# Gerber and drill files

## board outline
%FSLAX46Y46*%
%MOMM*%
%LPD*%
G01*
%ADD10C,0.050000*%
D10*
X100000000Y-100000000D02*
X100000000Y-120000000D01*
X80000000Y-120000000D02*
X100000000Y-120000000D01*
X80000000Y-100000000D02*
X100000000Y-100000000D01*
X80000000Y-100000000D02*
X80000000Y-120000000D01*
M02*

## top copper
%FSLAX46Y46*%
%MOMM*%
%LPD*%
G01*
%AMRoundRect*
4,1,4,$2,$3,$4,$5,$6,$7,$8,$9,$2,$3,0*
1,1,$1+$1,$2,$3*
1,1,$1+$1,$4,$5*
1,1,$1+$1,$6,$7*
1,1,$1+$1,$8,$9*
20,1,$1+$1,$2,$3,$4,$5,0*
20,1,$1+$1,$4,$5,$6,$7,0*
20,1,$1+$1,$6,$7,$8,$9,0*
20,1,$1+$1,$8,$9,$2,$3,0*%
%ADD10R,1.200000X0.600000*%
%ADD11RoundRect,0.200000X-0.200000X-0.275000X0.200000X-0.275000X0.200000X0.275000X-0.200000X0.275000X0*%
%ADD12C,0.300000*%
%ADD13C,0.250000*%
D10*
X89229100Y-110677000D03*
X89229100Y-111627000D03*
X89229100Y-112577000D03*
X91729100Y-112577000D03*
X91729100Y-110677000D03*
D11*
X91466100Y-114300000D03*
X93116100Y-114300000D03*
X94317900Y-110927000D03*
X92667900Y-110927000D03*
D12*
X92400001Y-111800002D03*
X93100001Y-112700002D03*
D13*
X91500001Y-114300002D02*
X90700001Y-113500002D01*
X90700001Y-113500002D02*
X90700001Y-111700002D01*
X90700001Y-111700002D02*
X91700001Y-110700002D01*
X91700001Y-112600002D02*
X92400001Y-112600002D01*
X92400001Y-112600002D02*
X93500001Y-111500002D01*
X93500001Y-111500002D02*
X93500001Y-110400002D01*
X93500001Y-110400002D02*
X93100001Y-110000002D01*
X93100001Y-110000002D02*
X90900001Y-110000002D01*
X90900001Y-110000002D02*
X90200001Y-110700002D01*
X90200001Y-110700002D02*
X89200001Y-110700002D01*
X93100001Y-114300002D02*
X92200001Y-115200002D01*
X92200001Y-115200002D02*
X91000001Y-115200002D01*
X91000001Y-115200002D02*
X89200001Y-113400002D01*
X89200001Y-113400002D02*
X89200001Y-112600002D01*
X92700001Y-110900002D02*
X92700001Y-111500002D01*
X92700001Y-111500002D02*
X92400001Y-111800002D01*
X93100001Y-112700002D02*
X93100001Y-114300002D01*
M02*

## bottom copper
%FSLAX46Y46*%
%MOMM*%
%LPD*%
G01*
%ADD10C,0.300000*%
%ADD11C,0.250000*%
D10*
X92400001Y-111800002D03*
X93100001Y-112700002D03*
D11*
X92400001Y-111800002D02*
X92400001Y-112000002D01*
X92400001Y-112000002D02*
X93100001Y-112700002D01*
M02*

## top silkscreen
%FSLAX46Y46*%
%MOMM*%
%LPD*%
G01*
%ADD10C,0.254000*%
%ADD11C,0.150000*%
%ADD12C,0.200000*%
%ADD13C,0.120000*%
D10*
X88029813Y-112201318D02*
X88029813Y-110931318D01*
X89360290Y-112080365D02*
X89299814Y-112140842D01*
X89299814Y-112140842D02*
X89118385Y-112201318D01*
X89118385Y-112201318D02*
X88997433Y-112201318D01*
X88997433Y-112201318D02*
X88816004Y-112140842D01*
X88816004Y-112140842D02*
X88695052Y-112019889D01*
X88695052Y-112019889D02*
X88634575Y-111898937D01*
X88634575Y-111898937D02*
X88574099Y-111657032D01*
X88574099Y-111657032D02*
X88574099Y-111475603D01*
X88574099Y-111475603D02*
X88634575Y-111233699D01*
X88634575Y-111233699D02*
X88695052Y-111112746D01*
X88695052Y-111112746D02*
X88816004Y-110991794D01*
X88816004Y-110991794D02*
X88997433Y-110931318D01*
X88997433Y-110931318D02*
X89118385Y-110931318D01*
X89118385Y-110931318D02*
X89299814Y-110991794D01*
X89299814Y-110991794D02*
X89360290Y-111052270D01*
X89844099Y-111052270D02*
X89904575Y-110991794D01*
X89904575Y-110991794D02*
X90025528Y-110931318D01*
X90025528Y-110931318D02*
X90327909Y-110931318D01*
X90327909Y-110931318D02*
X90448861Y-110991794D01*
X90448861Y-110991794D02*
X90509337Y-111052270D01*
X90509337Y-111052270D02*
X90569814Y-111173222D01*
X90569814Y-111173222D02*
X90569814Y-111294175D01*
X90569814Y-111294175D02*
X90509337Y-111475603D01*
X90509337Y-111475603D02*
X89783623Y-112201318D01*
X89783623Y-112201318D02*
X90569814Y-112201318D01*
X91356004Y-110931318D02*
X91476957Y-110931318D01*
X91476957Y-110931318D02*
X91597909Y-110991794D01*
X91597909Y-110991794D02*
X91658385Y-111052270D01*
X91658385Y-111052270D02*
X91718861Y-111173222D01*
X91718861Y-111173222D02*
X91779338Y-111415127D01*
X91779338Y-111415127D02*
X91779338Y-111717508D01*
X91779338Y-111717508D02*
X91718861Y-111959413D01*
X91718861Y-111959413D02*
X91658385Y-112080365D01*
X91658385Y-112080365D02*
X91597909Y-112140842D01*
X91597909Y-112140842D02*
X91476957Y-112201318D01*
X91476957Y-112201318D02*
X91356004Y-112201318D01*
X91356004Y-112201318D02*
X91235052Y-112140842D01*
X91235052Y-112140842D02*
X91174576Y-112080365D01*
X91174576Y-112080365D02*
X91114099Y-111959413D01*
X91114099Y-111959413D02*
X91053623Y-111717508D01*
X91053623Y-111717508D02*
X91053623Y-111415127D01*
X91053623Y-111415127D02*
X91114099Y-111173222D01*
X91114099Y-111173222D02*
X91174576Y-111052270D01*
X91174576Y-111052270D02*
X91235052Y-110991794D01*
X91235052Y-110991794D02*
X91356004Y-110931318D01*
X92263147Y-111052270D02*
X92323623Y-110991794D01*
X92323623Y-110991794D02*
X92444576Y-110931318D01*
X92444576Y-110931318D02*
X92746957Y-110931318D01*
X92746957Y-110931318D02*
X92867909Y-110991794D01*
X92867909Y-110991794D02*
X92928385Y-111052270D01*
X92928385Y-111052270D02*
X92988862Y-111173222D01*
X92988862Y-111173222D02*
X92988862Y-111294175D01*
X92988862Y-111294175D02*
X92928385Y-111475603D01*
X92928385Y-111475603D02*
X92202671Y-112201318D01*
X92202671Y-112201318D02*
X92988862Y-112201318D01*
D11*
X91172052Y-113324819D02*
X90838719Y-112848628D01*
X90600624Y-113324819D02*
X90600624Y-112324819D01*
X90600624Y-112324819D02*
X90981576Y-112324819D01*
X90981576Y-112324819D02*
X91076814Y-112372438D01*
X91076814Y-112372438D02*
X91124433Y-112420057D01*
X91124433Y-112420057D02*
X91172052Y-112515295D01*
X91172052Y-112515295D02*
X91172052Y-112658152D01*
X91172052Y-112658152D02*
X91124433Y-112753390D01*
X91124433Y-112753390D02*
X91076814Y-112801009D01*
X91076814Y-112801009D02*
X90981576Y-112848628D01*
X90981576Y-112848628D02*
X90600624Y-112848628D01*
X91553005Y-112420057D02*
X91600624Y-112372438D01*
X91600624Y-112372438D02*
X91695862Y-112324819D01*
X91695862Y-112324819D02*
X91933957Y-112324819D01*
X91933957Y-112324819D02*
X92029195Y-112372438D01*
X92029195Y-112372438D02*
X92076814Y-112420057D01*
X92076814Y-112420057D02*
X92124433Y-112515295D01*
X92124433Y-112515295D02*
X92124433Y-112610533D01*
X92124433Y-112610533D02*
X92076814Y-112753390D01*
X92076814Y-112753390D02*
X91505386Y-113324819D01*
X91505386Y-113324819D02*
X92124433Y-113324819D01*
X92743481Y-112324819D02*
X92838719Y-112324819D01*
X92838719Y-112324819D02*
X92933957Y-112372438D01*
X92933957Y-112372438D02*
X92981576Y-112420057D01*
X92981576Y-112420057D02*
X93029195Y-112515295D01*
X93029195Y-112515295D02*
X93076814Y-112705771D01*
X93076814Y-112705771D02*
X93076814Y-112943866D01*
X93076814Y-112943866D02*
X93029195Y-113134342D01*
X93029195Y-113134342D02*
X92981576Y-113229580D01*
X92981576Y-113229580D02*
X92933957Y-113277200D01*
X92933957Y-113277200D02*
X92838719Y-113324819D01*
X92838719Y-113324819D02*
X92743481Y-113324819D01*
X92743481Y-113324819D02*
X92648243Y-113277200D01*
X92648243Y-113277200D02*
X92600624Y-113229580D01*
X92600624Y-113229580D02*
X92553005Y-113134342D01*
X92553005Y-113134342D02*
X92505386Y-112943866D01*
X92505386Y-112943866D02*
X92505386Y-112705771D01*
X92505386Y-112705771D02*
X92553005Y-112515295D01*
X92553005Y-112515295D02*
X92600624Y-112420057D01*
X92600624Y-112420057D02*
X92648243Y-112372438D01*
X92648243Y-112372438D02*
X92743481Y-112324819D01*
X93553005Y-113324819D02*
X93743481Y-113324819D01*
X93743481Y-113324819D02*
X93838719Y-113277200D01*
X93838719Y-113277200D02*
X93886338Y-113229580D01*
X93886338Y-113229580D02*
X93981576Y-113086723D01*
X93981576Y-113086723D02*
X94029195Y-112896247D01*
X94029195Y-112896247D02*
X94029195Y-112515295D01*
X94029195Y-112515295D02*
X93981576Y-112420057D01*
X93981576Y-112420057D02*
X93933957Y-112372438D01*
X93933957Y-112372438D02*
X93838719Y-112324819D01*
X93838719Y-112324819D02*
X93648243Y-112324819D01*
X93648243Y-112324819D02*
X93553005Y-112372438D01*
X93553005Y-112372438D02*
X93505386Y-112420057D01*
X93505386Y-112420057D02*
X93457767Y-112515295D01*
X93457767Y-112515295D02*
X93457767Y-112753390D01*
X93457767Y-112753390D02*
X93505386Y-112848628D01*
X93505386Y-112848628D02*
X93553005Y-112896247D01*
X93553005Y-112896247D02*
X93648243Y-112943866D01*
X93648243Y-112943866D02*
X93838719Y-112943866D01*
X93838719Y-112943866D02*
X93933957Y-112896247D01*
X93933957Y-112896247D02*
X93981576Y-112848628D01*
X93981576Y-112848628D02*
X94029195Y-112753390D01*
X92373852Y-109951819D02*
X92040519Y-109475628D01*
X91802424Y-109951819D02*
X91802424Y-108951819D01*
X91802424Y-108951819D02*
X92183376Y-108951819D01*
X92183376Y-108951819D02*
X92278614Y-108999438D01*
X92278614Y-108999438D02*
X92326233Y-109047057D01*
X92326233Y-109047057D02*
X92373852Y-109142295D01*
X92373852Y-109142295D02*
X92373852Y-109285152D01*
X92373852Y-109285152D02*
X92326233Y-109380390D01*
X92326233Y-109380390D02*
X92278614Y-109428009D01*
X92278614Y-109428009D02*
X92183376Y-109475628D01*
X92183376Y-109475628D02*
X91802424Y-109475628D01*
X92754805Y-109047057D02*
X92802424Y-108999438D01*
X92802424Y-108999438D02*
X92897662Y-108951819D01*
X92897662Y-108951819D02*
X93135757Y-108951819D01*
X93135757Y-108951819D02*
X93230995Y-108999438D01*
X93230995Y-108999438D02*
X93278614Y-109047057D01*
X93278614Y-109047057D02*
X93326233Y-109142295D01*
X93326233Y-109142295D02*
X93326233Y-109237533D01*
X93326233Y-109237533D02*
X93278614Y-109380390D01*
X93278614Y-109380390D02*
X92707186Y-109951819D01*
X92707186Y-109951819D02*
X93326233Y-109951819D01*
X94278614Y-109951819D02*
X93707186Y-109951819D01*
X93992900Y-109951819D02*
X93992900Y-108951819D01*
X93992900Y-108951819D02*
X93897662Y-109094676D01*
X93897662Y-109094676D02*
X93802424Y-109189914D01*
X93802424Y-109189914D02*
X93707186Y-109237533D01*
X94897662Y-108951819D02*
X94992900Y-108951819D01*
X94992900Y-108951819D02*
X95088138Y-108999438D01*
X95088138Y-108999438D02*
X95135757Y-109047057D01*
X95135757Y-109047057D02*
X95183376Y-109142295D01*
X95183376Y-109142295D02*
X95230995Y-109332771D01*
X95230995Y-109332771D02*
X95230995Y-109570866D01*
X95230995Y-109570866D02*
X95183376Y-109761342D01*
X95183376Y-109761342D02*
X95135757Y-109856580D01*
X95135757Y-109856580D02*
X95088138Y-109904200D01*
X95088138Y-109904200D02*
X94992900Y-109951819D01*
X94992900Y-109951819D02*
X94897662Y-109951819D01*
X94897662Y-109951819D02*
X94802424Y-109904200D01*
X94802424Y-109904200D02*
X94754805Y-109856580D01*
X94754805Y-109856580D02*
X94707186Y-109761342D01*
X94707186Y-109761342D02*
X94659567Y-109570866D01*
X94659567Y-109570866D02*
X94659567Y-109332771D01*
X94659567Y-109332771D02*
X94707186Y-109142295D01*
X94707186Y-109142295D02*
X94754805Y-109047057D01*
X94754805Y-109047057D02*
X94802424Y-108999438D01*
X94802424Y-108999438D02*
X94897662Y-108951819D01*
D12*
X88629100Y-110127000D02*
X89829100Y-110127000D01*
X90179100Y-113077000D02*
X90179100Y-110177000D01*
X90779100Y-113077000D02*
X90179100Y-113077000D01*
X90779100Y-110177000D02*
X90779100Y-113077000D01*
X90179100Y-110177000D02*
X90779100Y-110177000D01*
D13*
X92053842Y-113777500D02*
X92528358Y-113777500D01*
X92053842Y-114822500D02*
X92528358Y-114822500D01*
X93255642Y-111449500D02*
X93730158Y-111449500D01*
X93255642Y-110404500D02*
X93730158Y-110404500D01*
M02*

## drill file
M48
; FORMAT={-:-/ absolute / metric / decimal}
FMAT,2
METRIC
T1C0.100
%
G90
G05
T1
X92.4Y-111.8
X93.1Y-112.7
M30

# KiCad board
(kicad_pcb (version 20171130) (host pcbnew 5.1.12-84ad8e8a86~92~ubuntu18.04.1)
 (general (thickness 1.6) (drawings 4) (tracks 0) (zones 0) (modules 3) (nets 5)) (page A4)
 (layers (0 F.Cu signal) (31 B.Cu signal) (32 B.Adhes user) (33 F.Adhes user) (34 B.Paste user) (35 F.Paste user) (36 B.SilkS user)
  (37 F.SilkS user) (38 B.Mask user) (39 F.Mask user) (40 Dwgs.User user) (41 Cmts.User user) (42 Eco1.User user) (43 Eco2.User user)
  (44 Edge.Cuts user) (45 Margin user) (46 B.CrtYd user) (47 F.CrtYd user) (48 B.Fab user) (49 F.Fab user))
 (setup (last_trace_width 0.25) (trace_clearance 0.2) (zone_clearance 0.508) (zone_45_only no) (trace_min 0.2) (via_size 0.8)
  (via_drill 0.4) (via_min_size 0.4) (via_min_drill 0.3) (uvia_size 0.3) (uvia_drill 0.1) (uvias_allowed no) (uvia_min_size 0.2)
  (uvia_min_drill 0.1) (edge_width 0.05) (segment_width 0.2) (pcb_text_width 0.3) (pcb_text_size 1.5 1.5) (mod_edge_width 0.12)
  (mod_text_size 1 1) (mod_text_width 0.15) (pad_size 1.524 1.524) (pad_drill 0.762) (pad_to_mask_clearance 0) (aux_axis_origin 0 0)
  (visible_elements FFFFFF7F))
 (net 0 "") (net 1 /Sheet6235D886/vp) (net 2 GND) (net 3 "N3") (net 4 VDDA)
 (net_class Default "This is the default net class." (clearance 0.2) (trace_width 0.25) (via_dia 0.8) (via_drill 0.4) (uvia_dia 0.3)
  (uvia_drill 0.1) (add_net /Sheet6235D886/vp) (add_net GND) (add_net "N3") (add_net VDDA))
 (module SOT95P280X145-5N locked (layer F.Cu) (at 90.479100 111.627000)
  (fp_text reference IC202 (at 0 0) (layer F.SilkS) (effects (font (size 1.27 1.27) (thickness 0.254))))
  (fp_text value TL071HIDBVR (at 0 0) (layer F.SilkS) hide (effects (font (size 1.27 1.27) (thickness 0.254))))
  (fp_line (start -1.85 -1.5) (end -0.65 -1.5) (layer F.SilkS) (width 0.2))
  (fp_line (start -0.3 1.45) (end -0.3 -1.45) (layer F.SilkS) (width 0.2))
  (fp_line (start 0.3 1.45) (end -0.3 1.45) (layer F.SilkS) (width 0.2))
  (fp_line (start 0.3 -1.45) (end 0.3 1.45) (layer F.SilkS) (width 0.2))
  (fp_line (start -0.3 -1.45) (end 0.3 -1.45) (layer F.SilkS) (width 0.2))
  (pad 1 smd rect (at -1.25 -0.95 90.000000) (size 0.6 1.2) (layers F.Cu F.Mask F.Paste) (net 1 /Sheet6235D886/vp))
  (pad 2 smd rect (at -1.25 0 90.000000) (size 0.6 1.2) (layers F.Cu F.Mask F.Paste) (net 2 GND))
  (pad 3 smd rect (at -1.25 0.95 90.000000) (size 0.6 1.2) (layers F.Cu F.Mask F.Paste) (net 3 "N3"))
  (pad 4 smd rect (at 1.25 0.95 90.000000) (size 0.6 1.2) (layers F.Cu F.Mask F.Paste) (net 1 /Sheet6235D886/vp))
  (pad 5 smd rect (at 1.25 -0.95 90.000000) (size 0.6 1.2) (layers F.Cu F.Mask F.Paste) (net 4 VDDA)))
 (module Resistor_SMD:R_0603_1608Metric (layer F.Cu) (at 92.291100 114.300000)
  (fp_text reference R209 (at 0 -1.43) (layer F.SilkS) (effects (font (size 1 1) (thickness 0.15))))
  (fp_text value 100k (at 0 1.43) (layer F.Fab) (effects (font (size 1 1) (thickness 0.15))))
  (fp_line (start -0.237258 -0.5225) (end 0.237258 -0.5225) (layer F.SilkS) (width 0.12))
  (fp_line (start -0.237258 0.5225) (end 0.237258 0.5225) (layer F.SilkS) (width 0.12))
  (pad 1 smd roundrect (at -0.825 0) (size 0.8 0.95) (layers F.Cu F.Mask F.Paste) (roundrect_rratio 0.25) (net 4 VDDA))
  (pad 2 smd roundrect (at 0.825 0) (size 0.8 0.95) (layers F.Cu F.Mask F.Paste) (roundrect_rratio 0.25) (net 3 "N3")))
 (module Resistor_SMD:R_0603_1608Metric (layer F.Cu) (at 93.492900 110.927000)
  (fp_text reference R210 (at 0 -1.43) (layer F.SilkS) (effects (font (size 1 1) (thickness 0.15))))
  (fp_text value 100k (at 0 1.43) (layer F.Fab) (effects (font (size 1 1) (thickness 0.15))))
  (fp_line (start -0.237258 0.5225) (end 0.237258 0.5225) (layer F.SilkS) (width 0.12))
  (fp_line (start -0.237258 -0.5225) (end 0.237258 -0.5225) (layer F.SilkS) (width 0.12))
  (pad 2 smd roundrect (at 0.825 0) (size 0.8 0.95) (layers F.Cu F.Mask F.Paste) (roundrect_rratio 0.25) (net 2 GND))
  (pad 1 smd roundrect (at -0.825 0) (size 0.8 0.95) (layers F.Cu F.Mask F.Paste) (roundrect_rratio 0.25) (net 3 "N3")))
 (gr_line (start 100 100) (end 100 120) (layer Edge.Cuts) (width 0.05))
 (gr_line (start 80 120) (end 100 120) (layer Edge.Cuts) (width 0.05))
 (gr_line (start 80 100) (end 100 100) (layer Edge.Cuts) (width 0.05))
 (gr_line (start 80 100) (end 80 120) (layer Edge.Cuts) (width 0.05))
 (segment (start 91.500001 114.300002) (end 90.700001 113.500002) (width 0.250000) (layer F.Cu) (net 4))
 (segment (start 90.700001 113.500002) (end 90.700001 111.700002) (width 0.250000) (layer F.Cu) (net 4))
 (segment (start 90.700001 111.700002) (end 91.700001 110.700002) (width 0.250000) (layer F.Cu) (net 4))
 (segment (start 91.700001 112.600002) (end 92.400001 112.600002) (width 0.250000) (layer F.Cu) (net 1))
 (segment (start 92.400001 112.600002) (end 93.500001 111.500002) (width 0.250000) (layer F.Cu) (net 1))
 (segment (start 93.500001 111.500002) (end 93.500001 110.400002) (width 0.250000) (layer F.Cu) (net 1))
 (segment (start 93.500001 110.400002) (end 93.100001 110.000002) (width 0.250000) (layer F.Cu) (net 1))
 (segment (start 93.100001 110.000002) (end 90.900001 110.000002) (width 0.250000) (layer F.Cu) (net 1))
 (segment (start 90.900001 110.000002) (end 90.200001 110.700002) (width 0.250000) (layer F.Cu) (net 1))
 (segment (start 90.200001 110.700002) (end 89.200001 110.700002) (width 0.250000) (layer F.Cu) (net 1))
 (segment (start 93.100001 114.300002) (end 92.200001 115.200002) (width 0.250000) (layer F.Cu) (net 3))
 (segment (start 92.200001 115.200002) (end 91.000001 115.200002) (width 0.250000) (layer F.Cu) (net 3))
 (segment (start 91.000001 115.200002) (end 89.200001 113.400002) (width 0.250000) (layer F.Cu) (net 3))
 (segment (start 89.200001 113.400002) (end 89.200001 112.600002) (width 0.250000) (layer F.Cu) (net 3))
 (segment (start 92.700001 110.900002) (end 92.700001 111.500002) (width 0.250000) (layer F.Cu) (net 3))
 (segment (start 92.700001 111.500002) (end 92.400001 111.800002) (width 0.250000) (layer F.Cu) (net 3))
 (segment (start 92.400001 111.800002) (end 92.400001 112.000002) (width 0.250000) (layer B.Cu) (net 3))
 (segment (start 92.400001 112.000002) (end 93.100001 112.700002) (width 0.250000) (layer B.Cu) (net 3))
 (segment (start 93.100001 112.700002) (end 93.100001 114.300002) (width 0.250000) (layer F.Cu) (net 3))
 (via micro (at 92.400001 111.800002) (size 0.300000) (drill 0.100000) (layers F.Cu B.Cu) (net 3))
 (via micro (at 93.100001 112.700002) (size 0.300000) (drill 0.100000) (layers F.Cu B.Cu) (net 3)))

